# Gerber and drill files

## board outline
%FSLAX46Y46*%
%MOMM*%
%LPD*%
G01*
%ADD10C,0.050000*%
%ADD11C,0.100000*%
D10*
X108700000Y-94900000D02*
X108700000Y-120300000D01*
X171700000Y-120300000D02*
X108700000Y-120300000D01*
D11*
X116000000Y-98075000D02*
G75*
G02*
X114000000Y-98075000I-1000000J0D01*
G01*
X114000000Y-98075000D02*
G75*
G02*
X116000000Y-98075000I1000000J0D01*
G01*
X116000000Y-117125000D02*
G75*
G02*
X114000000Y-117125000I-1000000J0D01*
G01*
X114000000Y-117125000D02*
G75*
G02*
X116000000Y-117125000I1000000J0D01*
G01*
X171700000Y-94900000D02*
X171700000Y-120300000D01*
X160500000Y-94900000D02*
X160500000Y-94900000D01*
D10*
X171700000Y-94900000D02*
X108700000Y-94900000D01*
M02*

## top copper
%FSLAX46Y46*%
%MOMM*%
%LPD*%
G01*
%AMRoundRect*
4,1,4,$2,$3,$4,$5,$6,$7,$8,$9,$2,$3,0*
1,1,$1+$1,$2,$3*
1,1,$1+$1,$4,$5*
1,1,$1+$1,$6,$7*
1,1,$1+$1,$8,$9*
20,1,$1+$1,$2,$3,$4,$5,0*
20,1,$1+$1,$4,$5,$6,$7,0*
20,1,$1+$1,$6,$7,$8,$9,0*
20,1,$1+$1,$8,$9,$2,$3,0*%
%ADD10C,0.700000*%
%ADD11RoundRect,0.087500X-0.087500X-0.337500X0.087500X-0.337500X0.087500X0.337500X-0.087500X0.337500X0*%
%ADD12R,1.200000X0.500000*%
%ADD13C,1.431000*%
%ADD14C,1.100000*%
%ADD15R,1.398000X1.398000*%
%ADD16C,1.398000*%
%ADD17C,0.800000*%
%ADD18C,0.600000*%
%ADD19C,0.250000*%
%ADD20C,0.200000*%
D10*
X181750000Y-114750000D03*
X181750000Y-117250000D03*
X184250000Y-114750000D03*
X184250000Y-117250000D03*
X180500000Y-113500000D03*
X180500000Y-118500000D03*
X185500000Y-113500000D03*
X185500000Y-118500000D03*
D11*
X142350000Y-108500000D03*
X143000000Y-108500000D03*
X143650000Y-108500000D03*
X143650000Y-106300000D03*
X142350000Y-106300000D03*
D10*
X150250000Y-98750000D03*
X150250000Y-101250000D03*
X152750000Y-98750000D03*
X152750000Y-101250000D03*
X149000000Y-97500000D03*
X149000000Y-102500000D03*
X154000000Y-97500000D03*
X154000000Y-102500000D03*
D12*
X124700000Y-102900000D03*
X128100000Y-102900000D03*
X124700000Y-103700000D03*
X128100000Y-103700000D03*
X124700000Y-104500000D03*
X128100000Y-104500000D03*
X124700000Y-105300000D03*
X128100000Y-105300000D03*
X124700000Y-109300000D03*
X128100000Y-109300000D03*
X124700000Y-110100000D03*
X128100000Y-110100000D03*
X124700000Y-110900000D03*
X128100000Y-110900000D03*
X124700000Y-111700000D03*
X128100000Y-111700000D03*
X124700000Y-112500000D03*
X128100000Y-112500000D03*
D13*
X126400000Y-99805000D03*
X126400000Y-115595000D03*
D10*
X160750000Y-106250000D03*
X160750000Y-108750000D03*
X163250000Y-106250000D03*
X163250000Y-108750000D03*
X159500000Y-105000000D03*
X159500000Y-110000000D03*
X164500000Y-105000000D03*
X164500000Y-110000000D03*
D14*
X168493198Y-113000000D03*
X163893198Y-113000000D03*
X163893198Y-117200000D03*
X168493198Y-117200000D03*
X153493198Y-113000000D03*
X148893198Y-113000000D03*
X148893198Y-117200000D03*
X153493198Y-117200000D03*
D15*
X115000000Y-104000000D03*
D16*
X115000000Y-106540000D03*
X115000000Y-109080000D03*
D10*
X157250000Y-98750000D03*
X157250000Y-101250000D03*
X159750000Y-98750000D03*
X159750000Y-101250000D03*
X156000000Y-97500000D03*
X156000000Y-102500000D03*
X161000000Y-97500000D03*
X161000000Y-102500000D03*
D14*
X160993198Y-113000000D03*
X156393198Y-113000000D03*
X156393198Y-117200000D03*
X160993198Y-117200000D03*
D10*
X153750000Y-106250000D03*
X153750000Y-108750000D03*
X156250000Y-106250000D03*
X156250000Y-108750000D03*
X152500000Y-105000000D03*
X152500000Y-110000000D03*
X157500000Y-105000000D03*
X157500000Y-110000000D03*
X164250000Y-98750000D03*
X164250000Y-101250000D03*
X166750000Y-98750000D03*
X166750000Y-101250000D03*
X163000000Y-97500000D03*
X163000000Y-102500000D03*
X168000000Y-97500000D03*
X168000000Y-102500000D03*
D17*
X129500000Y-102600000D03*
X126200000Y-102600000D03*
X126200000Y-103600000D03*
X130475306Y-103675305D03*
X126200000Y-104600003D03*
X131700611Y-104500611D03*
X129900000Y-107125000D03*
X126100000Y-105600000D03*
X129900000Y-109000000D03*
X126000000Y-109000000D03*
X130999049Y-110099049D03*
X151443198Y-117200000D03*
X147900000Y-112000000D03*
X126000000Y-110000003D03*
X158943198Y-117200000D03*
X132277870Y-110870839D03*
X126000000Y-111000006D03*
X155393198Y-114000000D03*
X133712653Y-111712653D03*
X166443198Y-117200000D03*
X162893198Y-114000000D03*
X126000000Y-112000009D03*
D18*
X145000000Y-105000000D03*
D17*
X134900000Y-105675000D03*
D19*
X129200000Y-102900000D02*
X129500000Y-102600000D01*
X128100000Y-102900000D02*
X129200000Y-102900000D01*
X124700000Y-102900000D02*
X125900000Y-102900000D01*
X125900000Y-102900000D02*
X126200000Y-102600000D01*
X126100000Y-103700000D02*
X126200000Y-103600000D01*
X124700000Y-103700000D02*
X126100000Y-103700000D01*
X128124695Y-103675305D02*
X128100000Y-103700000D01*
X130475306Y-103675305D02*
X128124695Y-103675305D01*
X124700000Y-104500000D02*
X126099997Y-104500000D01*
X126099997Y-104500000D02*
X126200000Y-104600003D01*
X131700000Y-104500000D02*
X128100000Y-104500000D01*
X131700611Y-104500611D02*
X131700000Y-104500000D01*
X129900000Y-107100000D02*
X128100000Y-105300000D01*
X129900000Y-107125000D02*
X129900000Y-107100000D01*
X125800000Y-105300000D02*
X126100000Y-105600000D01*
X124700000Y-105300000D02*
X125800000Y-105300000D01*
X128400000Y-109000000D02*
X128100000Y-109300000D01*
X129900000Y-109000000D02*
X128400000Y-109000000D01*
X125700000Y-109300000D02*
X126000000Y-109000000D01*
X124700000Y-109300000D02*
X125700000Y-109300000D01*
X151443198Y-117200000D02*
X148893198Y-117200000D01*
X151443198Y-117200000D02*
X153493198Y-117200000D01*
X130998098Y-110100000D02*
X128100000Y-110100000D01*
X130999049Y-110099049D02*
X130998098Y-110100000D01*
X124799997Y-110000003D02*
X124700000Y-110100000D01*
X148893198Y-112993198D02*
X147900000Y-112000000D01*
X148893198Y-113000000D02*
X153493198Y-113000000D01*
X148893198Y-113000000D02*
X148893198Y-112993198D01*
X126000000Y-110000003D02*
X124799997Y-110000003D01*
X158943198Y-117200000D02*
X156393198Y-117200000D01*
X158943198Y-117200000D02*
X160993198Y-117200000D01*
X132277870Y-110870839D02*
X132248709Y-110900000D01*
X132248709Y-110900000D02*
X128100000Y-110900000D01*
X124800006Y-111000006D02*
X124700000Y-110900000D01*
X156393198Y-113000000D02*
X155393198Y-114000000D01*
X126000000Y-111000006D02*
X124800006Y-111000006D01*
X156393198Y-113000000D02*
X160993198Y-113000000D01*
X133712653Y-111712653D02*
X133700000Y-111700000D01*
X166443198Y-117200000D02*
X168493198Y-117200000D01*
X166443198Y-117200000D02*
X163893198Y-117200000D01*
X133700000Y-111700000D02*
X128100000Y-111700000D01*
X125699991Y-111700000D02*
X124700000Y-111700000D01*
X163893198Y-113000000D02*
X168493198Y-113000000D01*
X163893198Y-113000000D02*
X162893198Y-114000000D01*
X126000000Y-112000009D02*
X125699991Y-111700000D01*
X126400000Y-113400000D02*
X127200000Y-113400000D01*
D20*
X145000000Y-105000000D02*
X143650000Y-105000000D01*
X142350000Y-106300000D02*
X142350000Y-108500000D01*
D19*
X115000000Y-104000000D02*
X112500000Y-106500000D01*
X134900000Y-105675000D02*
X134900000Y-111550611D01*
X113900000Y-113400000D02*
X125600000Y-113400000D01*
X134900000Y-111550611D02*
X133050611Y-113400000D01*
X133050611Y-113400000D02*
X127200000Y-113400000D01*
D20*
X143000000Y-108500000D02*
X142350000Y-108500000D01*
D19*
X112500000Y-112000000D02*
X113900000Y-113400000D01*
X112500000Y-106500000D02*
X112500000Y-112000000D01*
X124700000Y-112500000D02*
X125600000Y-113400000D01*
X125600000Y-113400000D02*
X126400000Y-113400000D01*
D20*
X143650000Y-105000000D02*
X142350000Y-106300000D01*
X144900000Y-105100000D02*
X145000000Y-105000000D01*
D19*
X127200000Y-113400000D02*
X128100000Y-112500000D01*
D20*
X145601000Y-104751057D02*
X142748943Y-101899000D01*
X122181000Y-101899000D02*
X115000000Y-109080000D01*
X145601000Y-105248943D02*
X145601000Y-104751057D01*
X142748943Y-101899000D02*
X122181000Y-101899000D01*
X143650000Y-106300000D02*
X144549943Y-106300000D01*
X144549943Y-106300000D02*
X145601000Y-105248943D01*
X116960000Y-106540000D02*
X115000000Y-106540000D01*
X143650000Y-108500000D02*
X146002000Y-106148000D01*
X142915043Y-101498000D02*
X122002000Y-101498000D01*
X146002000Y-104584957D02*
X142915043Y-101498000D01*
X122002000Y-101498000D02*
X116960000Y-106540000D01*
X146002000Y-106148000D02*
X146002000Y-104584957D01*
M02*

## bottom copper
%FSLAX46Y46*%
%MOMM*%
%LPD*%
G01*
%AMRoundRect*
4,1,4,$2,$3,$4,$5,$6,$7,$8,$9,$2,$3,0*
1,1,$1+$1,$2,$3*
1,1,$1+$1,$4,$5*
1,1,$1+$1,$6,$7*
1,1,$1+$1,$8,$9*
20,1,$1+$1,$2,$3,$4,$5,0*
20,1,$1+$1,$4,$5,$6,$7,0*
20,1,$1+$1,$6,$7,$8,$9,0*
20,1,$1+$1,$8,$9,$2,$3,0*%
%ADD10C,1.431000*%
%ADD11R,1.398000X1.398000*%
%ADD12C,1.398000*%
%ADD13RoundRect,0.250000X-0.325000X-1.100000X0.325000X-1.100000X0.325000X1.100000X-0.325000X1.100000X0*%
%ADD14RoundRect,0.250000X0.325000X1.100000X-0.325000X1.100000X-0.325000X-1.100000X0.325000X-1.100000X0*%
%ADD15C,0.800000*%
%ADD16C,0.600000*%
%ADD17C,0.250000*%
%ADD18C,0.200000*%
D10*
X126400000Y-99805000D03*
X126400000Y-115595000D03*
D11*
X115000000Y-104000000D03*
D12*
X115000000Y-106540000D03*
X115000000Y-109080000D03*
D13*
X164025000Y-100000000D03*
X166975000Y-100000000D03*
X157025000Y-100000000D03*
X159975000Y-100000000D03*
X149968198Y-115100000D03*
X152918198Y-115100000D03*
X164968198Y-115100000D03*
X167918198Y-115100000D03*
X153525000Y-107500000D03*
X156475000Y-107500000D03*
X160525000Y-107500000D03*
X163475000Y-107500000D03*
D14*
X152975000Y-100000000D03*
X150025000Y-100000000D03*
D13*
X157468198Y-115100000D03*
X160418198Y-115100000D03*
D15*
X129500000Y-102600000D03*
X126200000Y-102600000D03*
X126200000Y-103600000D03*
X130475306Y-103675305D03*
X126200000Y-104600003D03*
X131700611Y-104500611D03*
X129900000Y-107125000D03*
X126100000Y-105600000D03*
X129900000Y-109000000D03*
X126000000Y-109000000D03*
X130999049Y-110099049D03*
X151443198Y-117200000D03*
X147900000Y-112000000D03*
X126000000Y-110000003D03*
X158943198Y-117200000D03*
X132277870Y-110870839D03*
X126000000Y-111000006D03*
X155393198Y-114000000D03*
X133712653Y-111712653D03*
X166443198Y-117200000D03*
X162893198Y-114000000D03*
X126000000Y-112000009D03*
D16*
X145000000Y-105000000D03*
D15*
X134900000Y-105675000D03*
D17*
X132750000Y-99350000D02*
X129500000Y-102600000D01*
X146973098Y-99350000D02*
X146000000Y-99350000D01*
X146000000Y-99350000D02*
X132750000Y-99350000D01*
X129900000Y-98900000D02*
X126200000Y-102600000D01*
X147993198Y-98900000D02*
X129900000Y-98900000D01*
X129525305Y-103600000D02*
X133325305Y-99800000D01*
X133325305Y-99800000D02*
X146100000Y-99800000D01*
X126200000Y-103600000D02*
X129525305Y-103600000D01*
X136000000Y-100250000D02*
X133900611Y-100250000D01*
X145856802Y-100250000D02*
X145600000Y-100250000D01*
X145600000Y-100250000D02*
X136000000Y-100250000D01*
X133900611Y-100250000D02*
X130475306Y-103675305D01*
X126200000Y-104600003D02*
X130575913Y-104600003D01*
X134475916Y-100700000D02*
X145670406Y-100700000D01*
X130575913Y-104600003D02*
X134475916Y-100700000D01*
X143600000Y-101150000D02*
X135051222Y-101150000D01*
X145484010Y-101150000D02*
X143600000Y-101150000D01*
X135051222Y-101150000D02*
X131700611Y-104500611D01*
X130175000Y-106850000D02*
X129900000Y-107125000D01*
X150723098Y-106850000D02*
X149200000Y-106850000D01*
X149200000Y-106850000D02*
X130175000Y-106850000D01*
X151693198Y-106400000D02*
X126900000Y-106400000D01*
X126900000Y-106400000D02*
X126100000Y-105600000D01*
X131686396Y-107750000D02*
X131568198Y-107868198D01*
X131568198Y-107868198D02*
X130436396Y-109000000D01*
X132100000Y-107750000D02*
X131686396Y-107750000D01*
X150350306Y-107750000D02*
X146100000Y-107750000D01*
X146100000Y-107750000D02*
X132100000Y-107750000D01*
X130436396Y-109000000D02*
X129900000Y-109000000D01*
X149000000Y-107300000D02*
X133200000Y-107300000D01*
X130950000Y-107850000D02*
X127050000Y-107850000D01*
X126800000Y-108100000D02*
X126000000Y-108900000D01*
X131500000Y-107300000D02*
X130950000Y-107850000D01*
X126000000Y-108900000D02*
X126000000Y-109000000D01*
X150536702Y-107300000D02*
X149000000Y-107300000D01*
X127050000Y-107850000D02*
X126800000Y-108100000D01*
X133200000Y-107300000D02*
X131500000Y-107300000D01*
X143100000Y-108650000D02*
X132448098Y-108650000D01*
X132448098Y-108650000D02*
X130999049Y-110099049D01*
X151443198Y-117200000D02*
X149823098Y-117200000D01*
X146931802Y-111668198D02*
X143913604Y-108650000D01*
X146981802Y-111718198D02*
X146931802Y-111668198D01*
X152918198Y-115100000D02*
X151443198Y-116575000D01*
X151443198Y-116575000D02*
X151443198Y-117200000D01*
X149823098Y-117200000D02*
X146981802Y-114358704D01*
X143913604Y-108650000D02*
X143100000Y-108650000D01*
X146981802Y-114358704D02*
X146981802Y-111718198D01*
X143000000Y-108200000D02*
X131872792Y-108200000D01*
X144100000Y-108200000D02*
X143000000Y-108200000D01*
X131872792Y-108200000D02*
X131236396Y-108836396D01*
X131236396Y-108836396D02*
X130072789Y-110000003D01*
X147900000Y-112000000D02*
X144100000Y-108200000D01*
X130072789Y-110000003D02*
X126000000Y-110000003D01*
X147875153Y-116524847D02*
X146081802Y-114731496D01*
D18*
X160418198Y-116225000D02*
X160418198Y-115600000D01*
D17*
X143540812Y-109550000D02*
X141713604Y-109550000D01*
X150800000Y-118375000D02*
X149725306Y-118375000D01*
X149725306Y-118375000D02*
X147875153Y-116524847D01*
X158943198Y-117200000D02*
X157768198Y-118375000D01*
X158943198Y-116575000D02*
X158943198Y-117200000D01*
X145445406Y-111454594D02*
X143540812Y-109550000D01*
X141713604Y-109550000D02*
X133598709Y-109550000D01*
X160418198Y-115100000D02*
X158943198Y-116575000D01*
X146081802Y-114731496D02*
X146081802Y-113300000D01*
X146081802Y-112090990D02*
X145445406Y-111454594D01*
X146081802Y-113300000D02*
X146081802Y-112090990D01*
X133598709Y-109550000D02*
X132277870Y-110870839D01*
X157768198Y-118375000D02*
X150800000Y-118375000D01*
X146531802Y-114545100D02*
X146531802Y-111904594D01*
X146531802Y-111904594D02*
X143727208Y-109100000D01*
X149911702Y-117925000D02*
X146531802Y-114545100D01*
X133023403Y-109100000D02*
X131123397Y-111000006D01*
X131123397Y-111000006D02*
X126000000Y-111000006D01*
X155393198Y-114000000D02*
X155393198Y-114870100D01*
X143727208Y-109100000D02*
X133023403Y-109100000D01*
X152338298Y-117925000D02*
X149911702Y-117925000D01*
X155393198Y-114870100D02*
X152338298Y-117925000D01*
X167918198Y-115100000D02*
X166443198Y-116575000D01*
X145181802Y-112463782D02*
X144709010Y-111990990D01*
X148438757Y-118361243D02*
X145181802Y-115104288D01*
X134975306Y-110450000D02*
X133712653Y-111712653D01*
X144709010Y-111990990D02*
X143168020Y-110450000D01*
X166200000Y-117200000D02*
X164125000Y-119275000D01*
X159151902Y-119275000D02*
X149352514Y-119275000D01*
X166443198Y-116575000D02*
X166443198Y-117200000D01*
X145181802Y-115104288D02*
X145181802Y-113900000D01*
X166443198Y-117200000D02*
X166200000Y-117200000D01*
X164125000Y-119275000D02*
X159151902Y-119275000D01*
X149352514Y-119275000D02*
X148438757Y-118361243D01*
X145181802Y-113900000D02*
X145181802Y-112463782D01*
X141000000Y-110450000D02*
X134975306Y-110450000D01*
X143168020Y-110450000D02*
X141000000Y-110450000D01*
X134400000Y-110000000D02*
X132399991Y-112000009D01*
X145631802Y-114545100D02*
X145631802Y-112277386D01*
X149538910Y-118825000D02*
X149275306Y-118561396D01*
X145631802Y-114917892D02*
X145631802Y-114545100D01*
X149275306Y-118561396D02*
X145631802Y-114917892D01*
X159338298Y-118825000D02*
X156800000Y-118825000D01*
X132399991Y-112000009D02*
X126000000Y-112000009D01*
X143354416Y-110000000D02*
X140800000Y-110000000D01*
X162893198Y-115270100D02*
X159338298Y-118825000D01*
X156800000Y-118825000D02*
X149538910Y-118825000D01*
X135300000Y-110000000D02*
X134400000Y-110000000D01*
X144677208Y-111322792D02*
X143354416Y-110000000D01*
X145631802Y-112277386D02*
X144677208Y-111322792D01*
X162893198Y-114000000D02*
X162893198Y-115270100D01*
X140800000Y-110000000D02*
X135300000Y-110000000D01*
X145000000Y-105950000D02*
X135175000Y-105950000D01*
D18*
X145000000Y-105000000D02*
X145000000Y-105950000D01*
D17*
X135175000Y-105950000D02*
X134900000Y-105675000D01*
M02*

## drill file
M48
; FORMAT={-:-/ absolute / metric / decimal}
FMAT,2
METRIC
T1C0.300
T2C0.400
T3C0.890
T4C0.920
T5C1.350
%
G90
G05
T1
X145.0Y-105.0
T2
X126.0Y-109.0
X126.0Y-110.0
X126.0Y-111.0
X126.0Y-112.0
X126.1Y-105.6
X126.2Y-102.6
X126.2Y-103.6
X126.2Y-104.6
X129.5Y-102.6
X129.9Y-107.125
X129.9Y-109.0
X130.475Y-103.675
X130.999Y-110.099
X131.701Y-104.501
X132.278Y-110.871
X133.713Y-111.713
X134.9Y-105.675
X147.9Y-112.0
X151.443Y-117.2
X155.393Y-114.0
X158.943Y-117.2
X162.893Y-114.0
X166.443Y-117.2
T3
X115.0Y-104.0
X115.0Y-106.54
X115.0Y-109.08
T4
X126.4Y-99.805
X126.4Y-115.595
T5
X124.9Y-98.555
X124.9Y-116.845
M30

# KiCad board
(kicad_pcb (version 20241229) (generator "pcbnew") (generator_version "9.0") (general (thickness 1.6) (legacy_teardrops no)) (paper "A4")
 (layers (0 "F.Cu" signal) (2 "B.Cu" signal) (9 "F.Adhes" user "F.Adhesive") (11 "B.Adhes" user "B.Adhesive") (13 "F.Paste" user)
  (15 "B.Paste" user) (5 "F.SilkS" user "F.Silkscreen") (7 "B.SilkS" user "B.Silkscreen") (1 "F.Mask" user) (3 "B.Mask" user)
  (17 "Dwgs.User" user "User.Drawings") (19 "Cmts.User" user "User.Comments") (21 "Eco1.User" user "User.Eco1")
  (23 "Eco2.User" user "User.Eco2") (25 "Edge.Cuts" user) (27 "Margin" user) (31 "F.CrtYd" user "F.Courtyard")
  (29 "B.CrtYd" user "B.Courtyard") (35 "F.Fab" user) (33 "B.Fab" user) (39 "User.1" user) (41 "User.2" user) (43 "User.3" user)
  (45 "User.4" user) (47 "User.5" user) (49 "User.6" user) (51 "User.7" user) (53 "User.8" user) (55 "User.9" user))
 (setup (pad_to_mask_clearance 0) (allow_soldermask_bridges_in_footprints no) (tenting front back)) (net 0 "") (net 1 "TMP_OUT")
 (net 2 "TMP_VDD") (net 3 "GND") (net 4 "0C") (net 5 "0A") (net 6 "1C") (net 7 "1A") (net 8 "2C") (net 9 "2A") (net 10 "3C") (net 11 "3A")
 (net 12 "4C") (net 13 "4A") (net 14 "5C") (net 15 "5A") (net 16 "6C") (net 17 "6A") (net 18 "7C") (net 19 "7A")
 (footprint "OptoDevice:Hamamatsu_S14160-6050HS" (layer "F.Cu") (at 183 116)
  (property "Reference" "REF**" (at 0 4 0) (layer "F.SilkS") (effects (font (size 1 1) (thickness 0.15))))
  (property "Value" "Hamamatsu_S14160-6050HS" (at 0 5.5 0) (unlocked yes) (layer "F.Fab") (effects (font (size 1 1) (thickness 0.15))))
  (pad "A" smd circle (at -1.25 -1.25) (size 0.7 0.7) (layers "F.Cu" "F.Mask" "F.Paste"))
  (pad "A" smd circle (at -1.25 1.25) (size 0.7 0.7) (layers "F.Cu" "F.Mask" "F.Paste"))
  (pad "A" smd circle (at 1.25 -1.25) (size 0.7 0.7) (layers "F.Cu" "F.Mask" "F.Paste"))
  (pad "A" smd circle (at 1.25 1.25) (size 0.7 0.7) (layers "F.Cu" "F.Mask" "F.Paste"))
  (pad "K" smd circle (at -2.5 -2.5) (size 0.7 0.7) (layers "F.Cu" "F.Mask" "F.Paste"))
  (pad "K" smd circle (at -2.5 2.5) (size 0.7 0.7) (layers "F.Cu" "F.Mask" "F.Paste"))
  (pad "K" smd circle (at 2.5 -2.5) (size 0.7 0.7) (layers "F.Cu" "F.Mask" "F.Paste"))
  (pad "K" smd circle (at 2.5 2.5) (size 0.7 0.7) (layers "F.Cu" "F.Mask" "F.Paste")))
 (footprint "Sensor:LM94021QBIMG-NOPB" (layer "F.Cu") (at 143 107.4)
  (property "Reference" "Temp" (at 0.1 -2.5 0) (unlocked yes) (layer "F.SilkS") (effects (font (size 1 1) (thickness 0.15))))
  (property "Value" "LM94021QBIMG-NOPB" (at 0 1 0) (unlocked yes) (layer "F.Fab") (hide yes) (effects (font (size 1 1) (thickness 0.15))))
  (pad "1" smd roundrect (at -0.65 1.1) (size 0.35 0.85) (layers "F.Cu" "F.Mask" "F.Paste") (roundrect_rratio 0.25))
  (pad "2" smd roundrect (at 0 1.1) (size 0.35 0.85) (layers "F.Cu" "F.Mask" "F.Paste") (roundrect_rratio 0.25))
  (pad "3" smd roundrect (at 0.65 1.1) (size 0.35 0.85) (layers "F.Cu" "F.Mask" "F.Paste") (roundrect_rratio 0.25) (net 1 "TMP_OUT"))
  (pad "4" smd roundrect (at 0.65 -1.1) (size 0.35 0.85) (layers "F.Cu" "F.Mask" "F.Paste") (roundrect_rratio 0.25) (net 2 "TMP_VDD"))
  (pad "5" smd roundrect (at -0.65 -1.1) (size 0.35 0.85) (layers "F.Cu" "F.Mask" "F.Paste") (roundrect_rratio 0.25) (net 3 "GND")))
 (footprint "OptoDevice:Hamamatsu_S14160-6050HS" (layer "F.Cu") (at 151.5 100)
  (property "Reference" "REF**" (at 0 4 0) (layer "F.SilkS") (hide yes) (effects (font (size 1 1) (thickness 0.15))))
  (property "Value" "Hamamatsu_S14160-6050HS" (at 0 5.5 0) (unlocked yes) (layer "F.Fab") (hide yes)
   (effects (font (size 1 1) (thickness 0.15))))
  (pad "A" smd circle (at -1.25 -1.25) (size 0.7 0.7) (layers "F.Cu" "F.Mask" "F.Paste"))
  (pad "A" smd circle (at -1.25 1.25) (size 0.7 0.7) (layers "F.Cu" "F.Mask" "F.Paste"))
  (pad "A" smd circle (at 1.25 -1.25) (size 0.7 0.7) (layers "F.Cu" "F.Mask" "F.Paste"))
  (pad "A" smd circle (at 1.25 1.25) (size 0.7 0.7) (layers "F.Cu" "F.Mask" "F.Paste"))
  (pad "K" smd circle (at -2.5 -2.5) (size 0.7 0.7) (layers "F.Cu" "F.Mask" "F.Paste"))
  (pad "K" smd circle (at -2.5 2.5) (size 0.7 0.7) (layers "F.Cu" "F.Mask" "F.Paste"))
  (pad "K" smd circle (at 2.5 -2.5) (size 0.7 0.7) (layers "F.Cu" "F.Mask" "F.Paste"))
  (pad "K" smd circle (at 2.5 2.5) (size 0.7 0.7) (layers "F.Cu" "F.Mask" "F.Paste")))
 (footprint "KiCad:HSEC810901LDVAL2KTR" (layer "F.Cu") (at 126.4 107.7 -90)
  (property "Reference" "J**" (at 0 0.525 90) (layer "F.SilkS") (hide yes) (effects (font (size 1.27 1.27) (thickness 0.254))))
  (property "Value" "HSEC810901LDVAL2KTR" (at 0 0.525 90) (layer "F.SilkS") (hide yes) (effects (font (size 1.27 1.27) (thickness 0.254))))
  (pad "" np_thru_hole circle (at -9.145 1.5 270) (size 1.35 1.35) (drill 1.35) (layers "*.Cu" "*.Mask"))
  (pad "" np_thru_hole circle (at 9.145 1.5 270) (size 1.35 1.35) (drill 1.35) (layers "*.Cu" "*.Mask"))
  (pad "1" smd rect (at -4.8 1.7 270) (size 0.5 1.2) (layers "F.Cu" "F.Mask" "F.Paste") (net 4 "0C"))
  (pad "2" smd rect (at -4.8 -1.7 270) (size 0.5 1.2) (layers "F.Cu" "F.Mask" "F.Paste") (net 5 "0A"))
  (pad "3" smd rect (at -4 1.7 270) (size 0.5 1.2) (layers "F.Cu" "F.Mask" "F.Paste") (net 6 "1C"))
  (pad "4" smd rect (at -4 -1.7 270) (size 0.5 1.2) (layers "F.Cu" "F.Mask" "F.Paste") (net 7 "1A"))
  (pad "5" smd rect (at -3.2 1.7 270) (size 0.5 1.2) (layers "F.Cu" "F.Mask" "F.Paste") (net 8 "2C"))
  (pad "6" smd rect (at -3.2 -1.7 270) (size 0.5 1.2) (layers "F.Cu" "F.Mask" "F.Paste") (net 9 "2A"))
  (pad "7" smd rect (at -2.4 1.7 270) (size 0.5 1.2) (layers "F.Cu" "F.Mask" "F.Paste") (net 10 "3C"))
  (pad "8" smd rect (at -2.4 -1.7 270) (size 0.5 1.2) (layers "F.Cu" "F.Mask" "F.Paste") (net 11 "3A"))
  (pad "9" smd rect (at 1.6 1.7 270) (size 0.5 1.2) (layers "F.Cu" "F.Mask" "F.Paste") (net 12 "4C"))
  (pad "10" smd rect (at 1.6 -1.7 270) (size 0.5 1.2) (layers "F.Cu" "F.Mask" "F.Paste") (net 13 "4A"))
  (pad "11" smd rect (at 2.4 1.7 270) (size 0.5 1.2) (layers "F.Cu" "F.Mask" "F.Paste") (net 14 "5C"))
  (pad "12" smd rect (at 2.4 -1.7 270) (size 0.5 1.2) (layers "F.Cu" "F.Mask" "F.Paste") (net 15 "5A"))
  (pad "13" smd rect (at 3.2 1.7 270) (size 0.5 1.2) (layers "F.Cu" "F.Mask" "F.Paste") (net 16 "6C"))
  (pad "14" smd rect (at 3.2 -1.7 270) (size 0.5 1.2) (layers "F.Cu" "F.Mask" "F.Paste") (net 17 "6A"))
  (pad "15" smd rect (at 4 1.7 270) (size 0.5 1.2) (layers "F.Cu" "F.Mask" "F.Paste") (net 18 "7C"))
  (pad "16" smd rect (at 4 -1.7 270) (size 0.5 1.2) (layers "F.Cu" "F.Mask" "F.Paste") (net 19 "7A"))
  (pad "17" smd rect (at 4.8 1.7 270) (size 0.5 1.2) (layers "F.Cu" "F.Mask" "F.Paste") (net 3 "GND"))
  (pad "18" smd rect (at 4.8 -1.7 270) (size 0.5 1.2) (layers "F.Cu" "F.Mask" "F.Paste") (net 3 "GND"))
  (pad "MH1" thru_hole circle (at -7.895 0 270) (size 1.431 1.431) (drill 0.92) (layers "*.Cu" "*.Mask") (remove_unused_layers no))
  (pad "MH2" thru_hole circle (at 7.895 0 270) (size 1.431 1.431) (drill 0.92) (layers "*.Cu" "*.Mask") (remove_unused_layers no)))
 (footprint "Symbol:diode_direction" (layer "F.Cu") (at 150.243198 107.6 90)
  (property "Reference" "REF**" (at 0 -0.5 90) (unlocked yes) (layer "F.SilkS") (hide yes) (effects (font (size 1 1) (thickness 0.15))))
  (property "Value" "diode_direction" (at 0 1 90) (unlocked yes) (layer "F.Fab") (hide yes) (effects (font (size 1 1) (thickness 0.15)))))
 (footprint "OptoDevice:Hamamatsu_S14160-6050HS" (layer "F.Cu") (at 162 107.5)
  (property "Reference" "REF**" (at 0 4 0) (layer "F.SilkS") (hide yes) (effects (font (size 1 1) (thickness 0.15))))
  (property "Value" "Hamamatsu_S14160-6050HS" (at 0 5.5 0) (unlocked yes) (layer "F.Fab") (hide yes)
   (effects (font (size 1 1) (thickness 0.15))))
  (pad "A" smd circle (at -1.25 -1.25) (size 0.7 0.7) (layers "F.Cu" "F.Mask" "F.Paste"))
  (pad "A" smd circle (at -1.25 1.25) (size 0.7 0.7) (layers "F.Cu" "F.Mask" "F.Paste"))
  (pad "A" smd circle (at 1.25 -1.25) (size 0.7 0.7) (layers "F.Cu" "F.Mask" "F.Paste"))
  (pad "A" smd circle (at 1.25 1.25) (size 0.7 0.7) (layers "F.Cu" "F.Mask" "F.Paste"))
  (pad "K" smd circle (at -2.5 -2.5) (size 0.7 0.7) (layers "F.Cu" "F.Mask" "F.Paste"))
  (pad "K" smd circle (at -2.5 2.5) (size 0.7 0.7) (layers "F.Cu" "F.Mask" "F.Paste"))
  (pad "K" smd circle (at 2.5 -2.5) (size 0.7 0.7) (layers "F.Cu" "F.Mask" "F.Paste"))
  (pad "K" smd circle (at 2.5 2.5) (size 0.7 0.7) (layers "F.Cu" "F.Mask" "F.Paste")))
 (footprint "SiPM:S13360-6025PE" (layer "F.Cu") (at 166.443198 115.1)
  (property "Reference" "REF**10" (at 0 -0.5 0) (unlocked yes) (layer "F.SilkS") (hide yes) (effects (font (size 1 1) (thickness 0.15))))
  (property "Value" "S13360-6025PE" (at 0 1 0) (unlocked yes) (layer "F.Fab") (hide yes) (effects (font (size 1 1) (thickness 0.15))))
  (pad "1" smd circle (at 2.05 -2.1) (size 1.1 1.1) (layers "F.Cu" "F.Mask" "F.Paste") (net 18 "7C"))
  (pad "2" smd circle (at -2.55 -2.1) (size 1.1 1.1) (layers "F.Cu" "F.Mask" "F.Paste") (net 18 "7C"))
  (pad "3" smd circle (at -2.55 2.1) (size 1.1 1.1) (layers "F.Cu" "F.Mask" "F.Paste") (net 19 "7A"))
  (pad "4" smd circle (at 2.05 2.1) (size 1.1 1.1) (layers "F.Cu" "F.Mask" "F.Paste") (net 19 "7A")))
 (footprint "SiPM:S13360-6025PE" (layer "F.Cu") (at 151.443198 115.1)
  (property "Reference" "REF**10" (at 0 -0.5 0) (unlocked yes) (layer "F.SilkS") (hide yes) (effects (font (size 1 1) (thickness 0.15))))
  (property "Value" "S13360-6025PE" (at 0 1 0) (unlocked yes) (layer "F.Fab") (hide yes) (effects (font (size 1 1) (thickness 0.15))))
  (pad "1" smd circle (at 2.05 -2.1) (size 1.1 1.1) (layers "F.Cu" "F.Mask" "F.Paste") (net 14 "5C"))
  (pad "2" smd circle (at -2.55 -2.1) (size 1.1 1.1) (layers "F.Cu" "F.Mask" "F.Paste") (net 14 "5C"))
  (pad "3" smd circle (at -2.55 2.1) (size 1.1 1.1) (layers "F.Cu" "F.Mask" "F.Paste") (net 15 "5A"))
  (pad "4" smd circle (at 2.05 2.1) (size 1.1 1.1) (layers "F.Cu" "F.Mask" "F.Paste") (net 15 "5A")))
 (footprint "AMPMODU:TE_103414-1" (layer "F.Cu") (at 115 106.54 -90)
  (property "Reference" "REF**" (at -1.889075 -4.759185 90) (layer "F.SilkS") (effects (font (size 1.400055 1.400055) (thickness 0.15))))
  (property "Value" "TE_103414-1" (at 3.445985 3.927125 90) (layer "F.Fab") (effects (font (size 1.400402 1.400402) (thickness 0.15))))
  (pad "1" thru_hole rect (at -2.54 0 270) (size 1.398 1.398) (drill 0.89) (layers "*.Cu" "*.Mask") (remove_unused_layers no) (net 3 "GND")
   (solder_mask_margin 0.102))
  (pad "2" thru_hole circle (at 0 0 270) (size 1.398 1.398) (drill 0.89) (layers "*.Cu" "*.Mask") (remove_unused_layers no)
   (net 1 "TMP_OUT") (solder_mask_margin 0.102))
  (pad "3" thru_hole circle (at 2.54 0 270) (size 1.398 1.398) (drill 0.89) (layers "*.Cu" "*.Mask") (remove_unused_layers no)
   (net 2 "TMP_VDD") (solder_mask_margin 0.102)))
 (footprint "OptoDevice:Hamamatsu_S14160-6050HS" (layer "F.Cu") (at 158.5 100)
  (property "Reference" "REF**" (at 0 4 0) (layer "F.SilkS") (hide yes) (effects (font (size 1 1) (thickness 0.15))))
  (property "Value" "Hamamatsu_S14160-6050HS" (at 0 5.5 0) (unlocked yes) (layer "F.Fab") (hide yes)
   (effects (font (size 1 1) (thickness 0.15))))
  (pad "A" smd circle (at -1.25 -1.25) (size 0.7 0.7) (layers "F.Cu" "F.Mask" "F.Paste"))
  (pad "A" smd circle (at -1.25 1.25) (size 0.7 0.7) (layers "F.Cu" "F.Mask" "F.Paste"))
  (pad "A" smd circle (at 1.25 -1.25) (size 0.7 0.7) (layers "F.Cu" "F.Mask" "F.Paste"))
  (pad "A" smd circle (at 1.25 1.25) (size 0.7 0.7) (layers "F.Cu" "F.Mask" "F.Paste"))
  (pad "K" smd circle (at -2.5 -2.5) (size 0.7 0.7) (layers "F.Cu" "F.Mask" "F.Paste"))
  (pad "K" smd circle (at -2.5 2.5) (size 0.7 0.7) (layers "F.Cu" "F.Mask" "F.Paste"))
  (pad "K" smd circle (at 2.5 -2.5) (size 0.7 0.7) (layers "F.Cu" "F.Mask" "F.Paste"))
  (pad "K" smd circle (at 2.5 2.5) (size 0.7 0.7) (layers "F.Cu" "F.Mask" "F.Paste")))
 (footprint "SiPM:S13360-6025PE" (layer "F.Cu") (at 158.943198 115.1)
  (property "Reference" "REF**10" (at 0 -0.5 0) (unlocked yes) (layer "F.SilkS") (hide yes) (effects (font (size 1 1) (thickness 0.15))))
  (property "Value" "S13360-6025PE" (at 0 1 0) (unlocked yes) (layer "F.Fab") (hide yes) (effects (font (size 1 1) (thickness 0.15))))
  (pad "1" smd circle (at 2.05 -2.1) (size 1.1 1.1) (layers "F.Cu" "F.Mask" "F.Paste") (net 16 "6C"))
  (pad "2" smd circle (at -2.55 -2.1) (size 1.1 1.1) (layers "F.Cu" "F.Mask" "F.Paste") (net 16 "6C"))
  (pad "3" smd circle (at -2.55 2.1) (size 1.1 1.1) (layers "F.Cu" "F.Mask" "F.Paste") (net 17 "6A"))
  (pad "4" smd circle (at 2.05 2.1) (size 1.1 1.1) (layers "F.Cu" "F.Mask" "F.Paste") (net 17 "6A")))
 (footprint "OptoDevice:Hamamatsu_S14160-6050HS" (layer "F.Cu") (at 155 107.5)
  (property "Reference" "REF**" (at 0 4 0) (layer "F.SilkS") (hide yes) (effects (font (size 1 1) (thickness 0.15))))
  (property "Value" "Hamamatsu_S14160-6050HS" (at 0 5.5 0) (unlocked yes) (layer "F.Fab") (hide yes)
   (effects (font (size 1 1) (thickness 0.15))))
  (pad "A" smd circle (at -1.25 -1.25) (size 0.7 0.7) (layers "F.Cu" "F.Mask" "F.Paste"))
  (pad "A" smd circle (at -1.25 1.25) (size 0.7 0.7) (layers "F.Cu" "F.Mask" "F.Paste"))
  (pad "A" smd circle (at 1.25 -1.25) (size 0.7 0.7) (layers "F.Cu" "F.Mask" "F.Paste"))
  (pad "A" smd circle (at 1.25 1.25) (size 0.7 0.7) (layers "F.Cu" "F.Mask" "F.Paste"))
  (pad "K" smd circle (at -2.5 -2.5) (size 0.7 0.7) (layers "F.Cu" "F.Mask" "F.Paste"))
  (pad "K" smd circle (at -2.5 2.5) (size 0.7 0.7) (layers "F.Cu" "F.Mask" "F.Paste"))
  (pad "K" smd circle (at 2.5 -2.5) (size 0.7 0.7) (layers "F.Cu" "F.Mask" "F.Paste"))
  (pad "K" smd circle (at 2.5 2.5) (size 0.7 0.7) (layers "F.Cu" "F.Mask" "F.Paste")))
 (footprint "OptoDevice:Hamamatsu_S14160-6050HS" (layer "F.Cu") (at 165.5 100)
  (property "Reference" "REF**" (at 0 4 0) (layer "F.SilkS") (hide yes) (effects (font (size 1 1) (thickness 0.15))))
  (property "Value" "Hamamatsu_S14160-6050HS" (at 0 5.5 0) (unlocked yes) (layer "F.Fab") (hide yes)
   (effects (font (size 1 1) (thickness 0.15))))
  (pad "A" smd circle (at -1.25 -1.25) (size 0.7 0.7) (layers "F.Cu" "F.Mask" "F.Paste"))
  (pad "A" smd circle (at -1.25 1.25) (size 0.7 0.7) (layers "F.Cu" "F.Mask" "F.Paste"))
  (pad "A" smd circle (at 1.25 -1.25) (size 0.7 0.7) (layers "F.Cu" "F.Mask" "F.Paste"))
  (pad "A" smd circle (at 1.25 1.25) (size 0.7 0.7) (layers "F.Cu" "F.Mask" "F.Paste"))
  (pad "K" smd circle (at -2.5 -2.5) (size 0.7 0.7) (layers "F.Cu" "F.Mask" "F.Paste"))
  (pad "K" smd circle (at -2.5 2.5) (size 0.7 0.7) (layers "F.Cu" "F.Mask" "F.Paste"))
  (pad "K" smd circle (at 2.5 -2.5) (size 0.7 0.7) (layers "F.Cu" "F.Mask" "F.Paste"))
  (pad "K" smd circle (at 2.5 2.5) (size 0.7 0.7) (layers "F.Cu" "F.Mask" "F.Paste")))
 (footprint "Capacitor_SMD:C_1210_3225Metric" (layer "B.Cu") (at 165.5 100)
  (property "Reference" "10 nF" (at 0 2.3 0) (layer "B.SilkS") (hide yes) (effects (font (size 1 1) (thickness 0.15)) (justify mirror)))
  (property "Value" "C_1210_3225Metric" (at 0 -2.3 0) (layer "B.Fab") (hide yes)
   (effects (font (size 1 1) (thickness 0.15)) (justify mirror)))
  (pad "1" smd roundrect (at -1.475 0) (size 1.15 2.7) (layers "B.Cu" "B.Mask" "B.Paste") (roundrect_rratio 0.2173913043) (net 3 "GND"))
  (pad "2" smd roundrect (at 1.475 0) (size 1.15 2.7) (layers "B.Cu" "B.Mask" "B.Paste") (roundrect_rratio 0.2173913043) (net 9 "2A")))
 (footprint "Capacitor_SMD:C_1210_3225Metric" (layer "B.Cu") (at 158.5 100)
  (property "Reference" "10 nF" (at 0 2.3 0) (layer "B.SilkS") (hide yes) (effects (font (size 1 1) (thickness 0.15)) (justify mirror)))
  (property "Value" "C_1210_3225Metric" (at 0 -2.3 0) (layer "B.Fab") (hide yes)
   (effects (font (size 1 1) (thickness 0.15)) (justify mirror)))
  (pad "1" smd roundrect (at -1.475 0) (size 1.15 2.7) (layers "B.Cu" "B.Mask" "B.Paste") (roundrect_rratio 0.2173913043) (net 3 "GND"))
  (pad "2" smd roundrect (at 1.475 0) (size 1.15 2.7) (layers "B.Cu" "B.Mask" "B.Paste") (roundrect_rratio 0.2173913043) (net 7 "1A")))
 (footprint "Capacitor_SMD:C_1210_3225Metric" (layer "B.Cu") (at 151.443198 115.1)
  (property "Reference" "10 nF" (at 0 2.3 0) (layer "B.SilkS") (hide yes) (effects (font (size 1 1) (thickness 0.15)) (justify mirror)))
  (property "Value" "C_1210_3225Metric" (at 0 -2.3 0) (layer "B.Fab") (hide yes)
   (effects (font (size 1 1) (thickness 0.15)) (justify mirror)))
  (pad "1" smd roundrect (at -1.475 0) (size 1.15 2.7) (layers "B.Cu" "B.Mask" "B.Paste") (roundrect_rratio 0.2173913043) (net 3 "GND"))
  (pad "2" smd roundrect (at 1.475 0) (size 1.15 2.7) (layers "B.Cu" "B.Mask" "B.Paste") (roundrect_rratio 0.2173913043) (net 15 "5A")))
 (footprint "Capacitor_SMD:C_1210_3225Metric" (layer "B.Cu") (at 166.443198 115.1)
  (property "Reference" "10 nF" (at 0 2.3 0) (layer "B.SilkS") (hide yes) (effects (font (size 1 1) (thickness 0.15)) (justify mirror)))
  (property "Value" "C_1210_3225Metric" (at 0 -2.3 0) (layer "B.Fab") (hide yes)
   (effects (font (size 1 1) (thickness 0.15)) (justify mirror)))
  (pad "1" smd roundrect (at -1.475 0) (size 1.15 2.7) (layers "B.Cu" "B.Mask" "B.Paste") (roundrect_rratio 0.2173913043) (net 3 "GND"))
  (pad "2" smd roundrect (at 1.475 0) (size 1.15 2.7) (layers "B.Cu" "B.Mask" "B.Paste") (roundrect_rratio 0.2173913043) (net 19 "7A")))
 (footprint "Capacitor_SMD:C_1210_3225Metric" (layer "B.Cu") (at 155 107.5)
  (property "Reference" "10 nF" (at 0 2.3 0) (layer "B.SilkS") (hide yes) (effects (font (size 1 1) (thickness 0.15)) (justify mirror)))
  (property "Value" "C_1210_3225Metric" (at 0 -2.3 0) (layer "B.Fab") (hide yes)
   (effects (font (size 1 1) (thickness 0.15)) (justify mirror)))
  (pad "1" smd roundrect (at -1.475 0) (size 1.15 2.7) (layers "B.Cu" "B.Mask" "B.Paste") (roundrect_rratio 0.2173913043) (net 3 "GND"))
  (pad "2" smd roundrect (at 1.475 0) (size 1.15 2.7) (layers "B.Cu" "B.Mask" "B.Paste") (roundrect_rratio 0.2173913043) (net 11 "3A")))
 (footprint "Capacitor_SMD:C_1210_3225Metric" (layer "B.Cu") (at 162 107.5)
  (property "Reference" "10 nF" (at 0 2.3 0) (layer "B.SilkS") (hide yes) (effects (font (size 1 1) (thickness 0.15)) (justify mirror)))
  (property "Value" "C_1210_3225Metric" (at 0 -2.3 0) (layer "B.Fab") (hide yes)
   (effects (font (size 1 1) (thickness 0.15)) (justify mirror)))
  (pad "1" smd roundrect (at -1.475 0) (size 1.15 2.7) (layers "B.Cu" "B.Mask" "B.Paste") (roundrect_rratio 0.2173913043) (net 3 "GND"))
  (pad "2" smd roundrect (at 1.475 0) (size 1.15 2.7) (layers "B.Cu" "B.Mask" "B.Paste") (roundrect_rratio 0.2173913043) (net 13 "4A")))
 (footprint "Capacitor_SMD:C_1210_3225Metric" (layer "B.Cu") (at 151.5 100 180)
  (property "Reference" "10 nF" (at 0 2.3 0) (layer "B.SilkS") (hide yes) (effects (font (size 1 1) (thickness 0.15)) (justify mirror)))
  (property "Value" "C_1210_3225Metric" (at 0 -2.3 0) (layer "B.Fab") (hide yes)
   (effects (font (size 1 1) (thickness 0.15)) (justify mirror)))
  (pad "1" smd roundrect (at -1.475 0 180) (size 1.15 2.7) (layers "B.Cu" "B.Mask" "B.Paste") (roundrect_rratio 0.2173913043) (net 5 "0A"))
  (pad "2" smd roundrect (at 1.475 0 180) (size 1.15 2.7) (layers "B.Cu" "B.Mask" "B.Paste") (roundrect_rratio 0.2173913043) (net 3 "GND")))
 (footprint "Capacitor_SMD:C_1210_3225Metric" (layer "B.Cu") (at 158.943198 115.1)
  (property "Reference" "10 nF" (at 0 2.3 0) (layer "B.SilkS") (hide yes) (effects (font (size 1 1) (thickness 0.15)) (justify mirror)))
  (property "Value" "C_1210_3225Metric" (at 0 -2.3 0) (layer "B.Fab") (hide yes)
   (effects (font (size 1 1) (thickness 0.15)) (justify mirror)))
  (pad "1" smd roundrect (at -1.475 0) (size 1.15 2.7) (layers "B.Cu" "B.Mask" "B.Paste") (roundrect_rratio 0.2173913043) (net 3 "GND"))
  (pad "2" smd roundrect (at 1.475 0) (size 1.15 2.7) (layers "B.Cu" "B.Mask" "B.Paste") (roundrect_rratio 0.2173913043) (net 17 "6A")))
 (gr_line (start 108.7 94.9) (end 108.7 120.3) (stroke (width 0.05) (type default)) (layer "Edge.Cuts"))
 (gr_line (start 171.7 120.3) (end 108.7 120.3) (stroke (width 0.05) (type solid)) (layer "Edge.Cuts"))
 (gr_circle (center 115 98.075) (end 116 98.075) (stroke (width 0.1) (type solid)) (fill no) (layer "Edge.Cuts"))
 (gr_circle (center 115 117.125) (end 116 117.125) (stroke (width 0.1) (type solid)) (fill no) (layer "Edge.Cuts"))
 (gr_line (start 171.7 94.9) (end 171.7 120.3) (stroke (width 0.1) (type default)) (layer "Edge.Cuts"))
 (gr_line (start 160.5 94.9) (end 160.5 94.9) (stroke (width 0.1) (type default)) (layer "Edge.Cuts"))
 (gr_line (start 171.7 94.9) (end 108.7 94.9) (stroke (width 0.05) (type solid)) (layer "Edge.Cuts"))
 (segment (start 129.2 102.9) (end 129.5 102.6) (width 0.25) (layer "F.Cu") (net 5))
 (segment (start 128.1 102.9) (end 129.2 102.9) (width 0.25) (layer "F.Cu") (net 5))
 (via (at 129.5 102.6) (size 0.8) (drill 0.4) (layers "F.Cu" "B.Cu") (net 5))
 (segment (start 132.75 99.35) (end 129.5 102.6) (width 0.25) (layer "B.Cu") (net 5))
 (segment (start 146.973098 99.35) (end 146 99.35) (width 0.25) (layer "B.Cu") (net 5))
 (segment (start 146 99.35) (end 132.75 99.35) (width 0.25) (layer "B.Cu") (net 5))
 (segment (start 124.7 102.9) (end 125.9 102.9) (width 0.25) (layer "F.Cu") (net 4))
 (segment (start 125.9 102.9) (end 126.2 102.6) (width 0.25) (layer "F.Cu") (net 4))
 (via (at 126.2 102.6) (size 0.8) (drill 0.4) (layers "F.Cu" "B.Cu") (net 4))
 (segment (start 129.9 98.9) (end 126.2 102.6) (width 0.25) (layer "B.Cu") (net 4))
 (segment (start 147.993198 98.9) (end 129.9 98.9) (width 0.25) (layer "B.Cu") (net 4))
 (segment (start 126.1 103.7) (end 126.2 103.6) (width 0.25) (layer "F.Cu") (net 6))
 (segment (start 124.7 103.7) (end 126.1 103.7) (width 0.25) (layer "F.Cu") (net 6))
 (via (at 126.2 103.6) (size 0.8) (drill 0.4) (layers "F.Cu" "B.Cu") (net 6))
 (segment (start 129.525305 103.6) (end 133.325305 99.8) (width 0.25) (layer "B.Cu") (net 6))
 (segment (start 133.325305 99.8) (end 146.1 99.8) (width 0.25) (layer "B.Cu") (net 6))
 (segment (start 126.2 103.6) (end 129.525305 103.6) (width 0.25) (layer "B.Cu") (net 6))
 (segment (start 128.124695 103.675305) (end 128.1 103.7) (width 0.25) (layer "F.Cu") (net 7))
 (segment (start 130.475306 103.675305) (end 128.124695 103.675305) (width 0.25) (layer "F.Cu") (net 7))
 (via (at 130.475306 103.675305) (size 0.8) (drill 0.4) (layers "F.Cu" "B.Cu") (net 7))
 (segment (start 136 100.25) (end 133.900611 100.25) (width 0.25) (layer "B.Cu") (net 7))
 (segment (start 145.856802 100.25) (end 145.6 100.25) (width 0.25) (layer "B.Cu") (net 7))
 (segment (start 145.6 100.25) (end 136 100.25) (width 0.25) (layer "B.Cu") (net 7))
 (segment (start 133.900611 100.25) (end 130.475306 103.675305) (width 0.25) (layer "B.Cu") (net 7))
 (segment (start 124.7 104.5) (end 126.099997 104.5) (width 0.25) (layer "F.Cu") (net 8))
 (segment (start 126.099997 104.5) (end 126.2 104.600003) (width 0.25) (layer "F.Cu") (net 8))
 (via (at 126.2 104.600003) (size 0.8) (drill 0.4) (layers "F.Cu" "B.Cu") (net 8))
 (segment (start 126.2 104.600003) (end 130.575913 104.600003) (width 0.25) (layer "B.Cu") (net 8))
 (segment (start 134.475916 100.7) (end 145.670406 100.7) (width 0.25) (layer "B.Cu") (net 8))
 (segment (start 130.575913 104.600003) (end 134.475916 100.7) (width 0.25) (layer "B.Cu") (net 8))
 (segment (start 131.7 104.5) (end 128.1 104.5) (width 0.25) (layer "F.Cu") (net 9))
 (segment (start 131.700611 104.500611) (end 131.7 104.5) (width 0.25) (layer "F.Cu") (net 9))
 (via (at 131.700611 104.500611) (size 0.8) (drill 0.4) (layers "F.Cu" "B.Cu") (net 9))
 (segment (start 143.6 101.15) (end 135.051222 101.15) (width 0.25) (layer "B.Cu") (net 9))
 (segment (start 145.48401 101.15) (end 143.6 101.15) (width 0.25) (layer "B.Cu") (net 9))
 (segment (start 135.051222 101.15) (end 131.700611 104.500611) (width 0.25) (layer "B.Cu") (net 9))
 (segment (start 129.9 107.1) (end 128.1 105.3) (width 0.25) (layer "F.Cu") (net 11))
 (segment (start 129.9 107.125) (end 129.9 107.1) (width 0.25) (layer "F.Cu") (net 11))
 (via (at 129.9 107.125) (size 0.8) (drill 0.4) (layers "F.Cu" "B.Cu") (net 11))
 (segment (start 130.175 106.85) (end 129.9 107.125) (width 0.25) (layer "B.Cu") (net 11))
 (segment (start 150.723098 106.85) (end 149.2 106.85) (width 0.25) (layer "B.Cu") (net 11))
 (segment (start 149.2 106.85) (end 130.175 106.85) (width 0.25) (layer "B.Cu") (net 11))
 (segment (start 125.8 105.3) (end 126.1 105.6) (width 0.25) (layer "F.Cu") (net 10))
 (segment (start 124.7 105.3) (end 125.8 105.3) (width 0.25) (layer "F.Cu") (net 10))
 (via (at 126.1 105.6) (size 0.8) (drill 0.4) (layers "F.Cu" "B.Cu") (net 10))
 (segment (start 151.693198 106.4) (end 126.9 106.4) (width 0.25) (layer "B.Cu") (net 10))
 (segment (start 126.9 106.4) (end 126.1 105.6) (width 0.25) (layer "B.Cu") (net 10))
 (segment (start 128.4 109) (end 128.1 109.3) (width 0.25) (layer "F.Cu") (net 13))
 (segment (start 129.9 109) (end 128.4 109) (width 0.25) (layer "F.Cu") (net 13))
 (via (at 129.9 109) (size 0.8) (drill 0.4) (layers "F.Cu" "B.Cu") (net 13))
 (segment (start 131.686396 107.75) (end 131.568198 107.868198) (width 0.25) (layer "B.Cu") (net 13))
 (segment (start 131.568198 107.868198) (end 130.436396 109) (width 0.25) (layer "B.Cu") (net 13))
 (segment (start 132.1 107.75) (end 131.686396 107.75) (width 0.25) (layer "B.Cu") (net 13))
 (segment (start 150.350306 107.75) (end 146.1 107.75) (width 0.25) (layer "B.Cu") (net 13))
 (segment (start 146.1 107.75) (end 132.1 107.75) (width 0.25) (layer "B.Cu") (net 13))
 (segment (start 130.436396 109) (end 129.9 109) (width 0.25) (layer "B.Cu") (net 13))
 (segment (start 125.7 109.3) (end 126 109) (width 0.25) (layer "F.Cu") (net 12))
 (segment (start 124.7 109.3) (end 125.7 109.3) (width 0.25) (layer "F.Cu") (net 12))
 (via (at 126 109) (size 0.8) (drill 0.4) (layers "F.Cu" "B.Cu") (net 12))
 (segment (start 149 107.3) (end 133.2 107.3) (width 0.25) (layer "B.Cu") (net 12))
 (segment (start 130.95 107.85) (end 127.05 107.85) (width 0.25) (layer "B.Cu") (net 12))
 (segment (start 126.8 108.1) (end 126 108.9) (width 0.25) (layer "B.Cu") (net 12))
 (segment (start 131.5 107.3) (end 130.95 107.85) (width 0.25) (layer "B.Cu") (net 12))
 (segment (start 126 108.9) (end 126 109) (width 0.25) (layer "B.Cu") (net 12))
 (segment (start 150.536702 107.3) (end 149 107.3) (width 0.25) (layer "B.Cu") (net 12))
 (segment (start 127.05 107.85) (end 126.8 108.1) (width 0.25) (layer "B.Cu") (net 12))
 (segment (start 133.2 107.3) (end 131.5 107.3) (width 0.25) (layer "B.Cu") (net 12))
 (segment (start 151.443198 117.2) (end 148.893198 117.2) (width 0.25) (layer "F.Cu") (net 15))
 (segment (start 151.443198 117.2) (end 153.493198 117.2) (width 0.25) (layer "F.Cu") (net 15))
 (segment (start 130.998098 110.1) (end 128.1 110.1) (width 0.25) (layer "F.Cu") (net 15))
 (segment (start 130.999049 110.099049) (end 130.998098 110.1) (width 0.25) (layer "F.Cu") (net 15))
 (via (at 130.999049 110.099049) (size 0.8) (drill 0.4) (layers "F.Cu" "B.Cu") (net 15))
 (via (at 151.443198 117.2) (size 0.8) (drill 0.4) (layers "F.Cu" "B.Cu") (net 15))
 (segment (start 143.1 108.65) (end 132.448098 108.65) (width 0.25) (layer "B.Cu") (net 15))
 (segment (start 132.448098 108.65) (end 130.999049 110.099049) (width 0.25) (layer "B.Cu") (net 15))
 (segment (start 151.443198 117.2) (end 149.823098 117.2) (width 0.25) (layer "B.Cu") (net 15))
 (segment (start 146.931802 111.668198) (end 143.913604 108.65) (width 0.25) (layer "B.Cu") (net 15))
 (segment (start 146.981802 111.718198) (end 146.931802 111.668198) (width 0.25) (layer "B.Cu") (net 15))
 (segment (start 152.918198 115.1) (end 151.443198 116.575) (width 0.25) (layer "B.Cu") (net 15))
 (segment (start 151.443198 116.575) (end 151.443198 117.2) (width 0.25) (layer "B.Cu") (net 15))
 (segment (start 149.823098 117.2) (end 146.981802 114.358704) (width 0.25) (layer "B.Cu") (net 15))
 (segment (start 143.913604 108.65) (end 143.1 108.65) (width 0.25) (layer "B.Cu") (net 15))
 (segment (start 146.981802 114.358704) (end 146.981802 111.718198) (width 0.25) (layer "B.Cu") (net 15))
 (segment (start 124.799997 110.000003) (end 124.7 110.1) (width 0.25) (layer "F.Cu") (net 14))
 (segment (start 148.893198 112.993198) (end 147.9 112) (width 0.25) (layer "F.Cu") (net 14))
 (segment (start 148.893198 113) (end 153.493198 113) (width 0.25) (layer "F.Cu") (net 14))
 (segment (start 148.893198 113) (end 148.893198 112.993198) (width 0.25) (layer "F.Cu") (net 14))
 (segment (start 126 110.000003) (end 124.799997 110.000003) (width 0.25) (layer "F.Cu") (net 14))
 (via (at 147.9 112) (size 0.8) (drill 0.4) (layers "F.Cu" "B.Cu") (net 14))
 (via (at 126 110.000003) (size 0.8) (drill 0.4) (layers "F.Cu" "B.Cu") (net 14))
 (segment (start 143 108.2) (end 131.872792 108.2) (width 0.25) (layer "B.Cu") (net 14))
 (segment (start 144.1 108.2) (end 143 108.2) (width 0.25) (layer "B.Cu") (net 14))
 (segment (start 131.872792 108.2) (end 131.236396 108.836396) (width 0.25) (layer "B.Cu") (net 14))
 (segment (start 131.236396 108.836396) (end 130.072789 110.000003) (width 0.25) (layer "B.Cu") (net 14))
 (segment (start 147.9 112) (end 144.1 108.2) (width 0.25) (layer "B.Cu") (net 14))
 (segment (start 130.072789 110.000003) (end 126 110.000003) (width 0.25) (layer "B.Cu") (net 14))
 (segment (start 158.943198 117.2) (end 156.393198 117.2) (width 0.25) (layer "F.Cu") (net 17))
 (segment (start 158.943198 117.2) (end 160.993198 117.2) (width 0.25) (layer "F.Cu") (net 17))
 (segment (start 132.27787 110.870839) (end 132.248709 110.9) (width 0.25) (layer "F.Cu") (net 17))
 (segment (start 132.248709 110.9) (end 128.1 110.9) (width 0.25) (layer "F.Cu") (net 17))
 (via (at 158.943198 117.2) (size 0.8) (drill 0.4) (layers "F.Cu" "B.Cu") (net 17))
 (via (at 132.27787 110.870839) (size 0.8) (drill 0.4) (layers "F.Cu" "B.Cu") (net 17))
 (segment (start 147.875153 116.524847) (end 146.081802 114.731496) (width 0.25) (layer "B.Cu") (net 17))
 (segment (start 160.418198 116.225) (end 160.418198 115.6) (width 0.2) (layer "B.Cu") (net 17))
 (segment (start 143.540812 109.55) (end 141.713604 109.55) (width 0.25) (layer "B.Cu") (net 17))
 (segment (start 150.8 118.375) (end 149.725306 118.375) (width 0.25) (layer "B.Cu") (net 17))
 (segment (start 149.725306 118.375) (end 147.875153 116.524847) (width 0.25) (layer "B.Cu") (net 17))
 (segment (start 158.943198 117.2) (end 157.768198 118.375) (width 0.25) (layer "B.Cu") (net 17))
 (segment (start 158.943198 116.575) (end 158.943198 117.2) (width 0.25) (layer "B.Cu") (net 17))
 (segment (start 145.445406 111.454594) (end 143.540812 109.55) (width 0.25) (layer "B.Cu") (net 17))
 (segment (start 141.713604 109.55) (end 133.598709 109.55) (width 0.25) (layer "B.Cu") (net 17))
 (segment (start 160.418198 115.1) (end 158.943198 116.575) (width 0.25) (layer "B.Cu") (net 17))
 (segment (start 146.081802 114.731496) (end 146.081802 113.3) (width 0.25) (layer "B.Cu") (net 17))
 (segment (start 146.081802 112.09099) (end 145.445406 111.454594) (width 0.25) (layer "B.Cu") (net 17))
 (segment (start 146.081802 113.3) (end 146.081802 112.09099) (width 0.25) (layer "B.Cu") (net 17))
 (segment (start 133.598709 109.55) (end 132.27787 110.870839) (width 0.25) (layer "B.Cu") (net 17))
 (segment (start 157.768198 118.375) (end 150.8 118.375) (width 0.25) (layer "B.Cu") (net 17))
 (segment (start 124.800006 111.000006) (end 124.7 110.9) (width 0.25) (layer "F.Cu") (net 16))
 (segment (start 156.393198 113) (end 155.393198 114) (width 0.25) (layer "F.Cu") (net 16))
 (segment (start 126 111.000006) (end 124.800006 111.000006) (width 0.25) (layer "F.Cu") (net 16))
 (segment (start 156.393198 113) (end 160.993198 113) (width 0.25) (layer "F.Cu") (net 16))
 (via (at 126 111.000006) (size 0.8) (drill 0.4) (layers "F.Cu" "B.Cu") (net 16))
 (via (at 155.393198 114) (size 0.8) (drill 0.4) (layers "F.Cu" "B.Cu") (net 16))
 (segment (start 146.531802 114.5451) (end 146.531802 111.904594) (width 0.25) (layer "B.Cu") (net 16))
 (segment (start 146.531802 111.904594) (end 143.727208 109.1) (width 0.25) (layer "B.Cu") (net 16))
 (segment (start 149.911702 117.925) (end 146.531802 114.5451) (width 0.25) (layer "B.Cu") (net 16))
 (segment (start 133.023403 109.1) (end 131.123397 111.000006) (width 0.25) (layer "B.Cu") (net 16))
 (segment (start 131.123397 111.000006) (end 126 111.000006) (width 0.25) (layer "B.Cu") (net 16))
 (segment (start 155.393198 114) (end 155.393198 114.8701) (width 0.25) (layer "B.Cu") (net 16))
 (segment (start 143.727208 109.1) (end 133.023403 109.1) (width 0.25) (layer "B.Cu") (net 16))
 (segment (start 152.338298 117.925) (end 149.911702 117.925) (width 0.25) (layer "B.Cu") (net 16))
 (segment (start 155.393198 114.8701) (end 152.338298 117.925) (width 0.25) (layer "B.Cu") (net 16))
 (segment (start 133.712653 111.712653) (end 133.7 111.7) (width 0.25) (layer "F.Cu") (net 19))
 (segment (start 166.443198 117.2) (end 168.493198 117.2) (width 0.25) (layer "F.Cu") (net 19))
 (segment (start 166.443198 117.2) (end 163.893198 117.2) (width 0.25) (layer "F.Cu") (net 19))
 (segment (start 133.7 111.7) (end 128.1 111.7) (width 0.25) (layer "F.Cu") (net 19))
 (via (at 133.712653 111.712653) (size 0.8) (drill 0.4) (layers "F.Cu" "B.Cu") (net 19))
 (via (at 166.443198 117.2) (size 0.8) (drill 0.4) (layers "F.Cu" "B.Cu") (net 19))
 (segment (start 167.918198 115.1) (end 166.443198 116.575) (width 0.25) (layer "B.Cu") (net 19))
 (segment (start 145.181802 112.463782) (end 144.70901 111.99099) (width 0.25) (layer "B.Cu") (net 19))
 (segment (start 148.438757 118.361243) (end 145.181802 115.104288) (width 0.25) (layer "B.Cu") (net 19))
 (segment (start 134.975306 110.45) (end 133.712653 111.712653) (width 0.25) (layer "B.Cu") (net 19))
 (segment (start 144.70901 111.99099) (end 143.16802 110.45) (width 0.25) (layer "B.Cu") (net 19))
 (segment (start 166.2 117.2) (end 164.125 119.275) (width 0.25) (layer "B.Cu") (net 19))
 (segment (start 159.151902 119.275) (end 149.352514 119.275) (width 0.25) (layer "B.Cu") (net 19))
 (segment (start 166.443198 116.575) (end 166.443198 117.2) (width 0.25) (layer "B.Cu") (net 19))
 (segment (start 145.181802 115.104288) (end 145.181802 113.9) (width 0.25) (layer "B.Cu") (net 19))
 (segment (start 166.443198 117.2) (end 166.2 117.2) (width 0.25) (layer "B.Cu") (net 19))
 (segment (start 164.125 119.275) (end 159.151902 119.275) (width 0.25) (layer "B.Cu") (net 19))
 (segment (start 149.352514 119.275) (end 148.438757 118.361243) (width 0.25) (layer "B.Cu") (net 19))
 (segment (start 145.181802 113.9) (end 145.181802 112.463782) (width 0.25) (layer "B.Cu") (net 19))
 (segment (start 141 110.45) (end 134.975306 110.45) (width 0.25) (layer "B.Cu") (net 19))
 (segment (start 143.16802 110.45) (end 141 110.45) (width 0.25) (layer "B.Cu") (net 19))
 (segment (start 125.699991 111.7) (end 124.7 111.7) (width 0.25) (layer "F.Cu") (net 18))
 (segment (start 163.893198 113) (end 168.493198 113) (width 0.25) (layer "F.Cu") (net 18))
 (segment (start 163.893198 113) (end 162.893198 114) (width 0.25) (layer "F.Cu") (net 18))
 (segment (start 126 112.000009) (end 125.699991 111.7) (width 0.25) (layer "F.Cu") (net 18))
 (via (at 162.893198 114) (size 0.8) (drill 0.4) (layers "F.Cu" "B.Cu") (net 18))
 (via (at 126 112.000009) (size 0.8) (drill 0.4) (layers "F.Cu" "B.Cu") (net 18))
 (segment (start 134.4 110) (end 132.399991 112.000009) (width 0.25) (layer "B.Cu") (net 18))
 (segment (start 145.631802 114.5451) (end 145.631802 112.277386) (width 0.25) (layer "B.Cu") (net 18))
 (segment (start 149.53891 118.825) (end 149.275306 118.561396) (width 0.25) (layer "B.Cu") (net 18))
 (segment (start 145.631802 114.917892) (end 145.631802 114.5451) (width 0.25) (layer "B.Cu") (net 18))
 (segment (start 149.275306 118.561396) (end 145.631802 114.917892) (width 0.25) (layer "B.Cu") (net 18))
 (segment (start 159.338298 118.825) (end 156.8 118.825) (width 0.25) (layer "B.Cu") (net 18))
 (segment (start 132.399991 112.000009) (end 126 112.000009) (width 0.25) (layer "B.Cu") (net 18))
 (segment (start 143.354416 110) (end 140.8 110) (width 0.25) (layer "B.Cu") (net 18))
 (segment (start 162.893198 115.2701) (end 159.338298 118.825) (width 0.25) (layer "B.Cu") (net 18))
 (segment (start 156.8 118.825) (end 149.53891 118.825) (width 0.25) (layer "B.Cu") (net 18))
 (segment (start 135.3 110) (end 134.4 110) (width 0.25) (layer "B.Cu") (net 18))
 (segment (start 144.677208 111.322792) (end 143.354416 110) (width 0.25) (layer "B.Cu") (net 18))
 (segment (start 145.631802 112.277386) (end 144.677208 111.322792) (width 0.25) (layer "B.Cu") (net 18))
 (segment (start 162.893198 114) (end 162.893198 115.2701) (width 0.25) (layer "B.Cu") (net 18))
 (segment (start 140.8 110) (end 135.3 110) (width 0.25) (layer "B.Cu") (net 18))
 (segment (start 126.4 113.4) (end 127.2 113.4) (width 0.25) (layer "F.Cu") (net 3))
 (segment (start 145 105) (end 143.65 105) (width 0.2) (layer "F.Cu") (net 3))
 (segment (start 142.35 106.3) (end 142.35 108.5) (width 0.2) (layer "F.Cu") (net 3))
 (segment (start 115 104) (end 112.5 106.5) (width 0.25) (layer "F.Cu") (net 3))
 (segment (start 134.9 105.675) (end 134.9 111.550611) (width 0.25) (layer "F.Cu") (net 3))
 (segment (start 113.9 113.4) (end 125.6 113.4) (width 0.25) (layer "F.Cu") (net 3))
 (segment (start 134.9 111.550611) (end 133.050611 113.4) (width 0.25) (layer "F.Cu") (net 3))
 (segment (start 133.050611 113.4) (end 127.2 113.4) (width 0.25) (layer "F.Cu") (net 3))
 (segment (start 143 108.5) (end 142.35 108.5) (width 0.2) (layer "F.Cu") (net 3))
 (segment (start 112.5 112) (end 113.9 113.4) (width 0.25) (layer "F.Cu") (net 3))
 (segment (start 112.5 106.5) (end 112.5 112) (width 0.25) (layer "F.Cu") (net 3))
 (segment (start 124.7 112.5) (end 125.6 113.4) (width 0.25) (layer "F.Cu") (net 3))
 (segment (start 125.6 113.4) (end 126.4 113.4) (width 0.25) (layer "F.Cu") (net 3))
 (segment (start 143.65 105) (end 142.35 106.3) (width 0.2) (layer "F.Cu") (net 3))
 (segment (start 144.9 105.1) (end 145 105) (width 0.2) (layer "F.Cu") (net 3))
 (segment (start 127.2 113.4) (end 128.1 112.5) (width 0.25) (layer "F.Cu") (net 3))
 (via (at 145 105) (size 0.6) (drill 0.3) (layers "F.Cu" "B.Cu") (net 3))
 (via (at 134.9 105.675) (size 0.8) (drill 0.4) (layers "F.Cu" "B.Cu") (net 3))
 (segment (start 145 105.95) (end 135.175 105.95) (width 0.25) (layer "B.Cu") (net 3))
 (segment (start 145 105) (end 145 105.95) (width 0.2) (layer "B.Cu") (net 3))
 (segment (start 135.175 105.95) (end 134.9 105.675) (width 0.25) (layer "B.Cu") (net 3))
 (segment (start 145.601 104.751057) (end 142.748943 101.899) (width 0.2) (layer "F.Cu") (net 2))
 (segment (start 122.181 101.899) (end 115 109.08) (width 0.2) (layer "F.Cu") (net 2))
 (segment (start 145.601 105.248943) (end 145.601 104.751057) (width 0.2) (layer "F.Cu") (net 2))
 (segment (start 142.748943 101.899) (end 122.181 101.899) (width 0.2) (layer "F.Cu") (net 2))
 (segment (start 143.65 106.3) (end 144.549943 106.3) (width 0.2) (layer "F.Cu") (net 2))
 (segment (start 144.549943 106.3) (end 145.601 105.248943) (width 0.2) (layer "F.Cu") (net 2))
 (segment (start 116.96 106.54) (end 115 106.54) (width 0.2) (layer "F.Cu") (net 1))
 (segment (start 143.65 108.5) (end 146.002 106.148) (width 0.2) (layer "F.Cu") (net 1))
 (segment (start 142.915043 101.498) (end 122.002 101.498) (width 0.2) (layer "F.Cu") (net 1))
 (segment (start 146.002 104.584957) (end 142.915043 101.498) (width 0.2) (layer "F.Cu") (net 1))
 (segment (start 122.002 101.498) (end 116.96 106.54) (width 0.2) (layer "F.Cu") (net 1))
 (segment (start 146.002 106.148) (end 146.002 104.584957) (width 0.2) (layer "F.Cu") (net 1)))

